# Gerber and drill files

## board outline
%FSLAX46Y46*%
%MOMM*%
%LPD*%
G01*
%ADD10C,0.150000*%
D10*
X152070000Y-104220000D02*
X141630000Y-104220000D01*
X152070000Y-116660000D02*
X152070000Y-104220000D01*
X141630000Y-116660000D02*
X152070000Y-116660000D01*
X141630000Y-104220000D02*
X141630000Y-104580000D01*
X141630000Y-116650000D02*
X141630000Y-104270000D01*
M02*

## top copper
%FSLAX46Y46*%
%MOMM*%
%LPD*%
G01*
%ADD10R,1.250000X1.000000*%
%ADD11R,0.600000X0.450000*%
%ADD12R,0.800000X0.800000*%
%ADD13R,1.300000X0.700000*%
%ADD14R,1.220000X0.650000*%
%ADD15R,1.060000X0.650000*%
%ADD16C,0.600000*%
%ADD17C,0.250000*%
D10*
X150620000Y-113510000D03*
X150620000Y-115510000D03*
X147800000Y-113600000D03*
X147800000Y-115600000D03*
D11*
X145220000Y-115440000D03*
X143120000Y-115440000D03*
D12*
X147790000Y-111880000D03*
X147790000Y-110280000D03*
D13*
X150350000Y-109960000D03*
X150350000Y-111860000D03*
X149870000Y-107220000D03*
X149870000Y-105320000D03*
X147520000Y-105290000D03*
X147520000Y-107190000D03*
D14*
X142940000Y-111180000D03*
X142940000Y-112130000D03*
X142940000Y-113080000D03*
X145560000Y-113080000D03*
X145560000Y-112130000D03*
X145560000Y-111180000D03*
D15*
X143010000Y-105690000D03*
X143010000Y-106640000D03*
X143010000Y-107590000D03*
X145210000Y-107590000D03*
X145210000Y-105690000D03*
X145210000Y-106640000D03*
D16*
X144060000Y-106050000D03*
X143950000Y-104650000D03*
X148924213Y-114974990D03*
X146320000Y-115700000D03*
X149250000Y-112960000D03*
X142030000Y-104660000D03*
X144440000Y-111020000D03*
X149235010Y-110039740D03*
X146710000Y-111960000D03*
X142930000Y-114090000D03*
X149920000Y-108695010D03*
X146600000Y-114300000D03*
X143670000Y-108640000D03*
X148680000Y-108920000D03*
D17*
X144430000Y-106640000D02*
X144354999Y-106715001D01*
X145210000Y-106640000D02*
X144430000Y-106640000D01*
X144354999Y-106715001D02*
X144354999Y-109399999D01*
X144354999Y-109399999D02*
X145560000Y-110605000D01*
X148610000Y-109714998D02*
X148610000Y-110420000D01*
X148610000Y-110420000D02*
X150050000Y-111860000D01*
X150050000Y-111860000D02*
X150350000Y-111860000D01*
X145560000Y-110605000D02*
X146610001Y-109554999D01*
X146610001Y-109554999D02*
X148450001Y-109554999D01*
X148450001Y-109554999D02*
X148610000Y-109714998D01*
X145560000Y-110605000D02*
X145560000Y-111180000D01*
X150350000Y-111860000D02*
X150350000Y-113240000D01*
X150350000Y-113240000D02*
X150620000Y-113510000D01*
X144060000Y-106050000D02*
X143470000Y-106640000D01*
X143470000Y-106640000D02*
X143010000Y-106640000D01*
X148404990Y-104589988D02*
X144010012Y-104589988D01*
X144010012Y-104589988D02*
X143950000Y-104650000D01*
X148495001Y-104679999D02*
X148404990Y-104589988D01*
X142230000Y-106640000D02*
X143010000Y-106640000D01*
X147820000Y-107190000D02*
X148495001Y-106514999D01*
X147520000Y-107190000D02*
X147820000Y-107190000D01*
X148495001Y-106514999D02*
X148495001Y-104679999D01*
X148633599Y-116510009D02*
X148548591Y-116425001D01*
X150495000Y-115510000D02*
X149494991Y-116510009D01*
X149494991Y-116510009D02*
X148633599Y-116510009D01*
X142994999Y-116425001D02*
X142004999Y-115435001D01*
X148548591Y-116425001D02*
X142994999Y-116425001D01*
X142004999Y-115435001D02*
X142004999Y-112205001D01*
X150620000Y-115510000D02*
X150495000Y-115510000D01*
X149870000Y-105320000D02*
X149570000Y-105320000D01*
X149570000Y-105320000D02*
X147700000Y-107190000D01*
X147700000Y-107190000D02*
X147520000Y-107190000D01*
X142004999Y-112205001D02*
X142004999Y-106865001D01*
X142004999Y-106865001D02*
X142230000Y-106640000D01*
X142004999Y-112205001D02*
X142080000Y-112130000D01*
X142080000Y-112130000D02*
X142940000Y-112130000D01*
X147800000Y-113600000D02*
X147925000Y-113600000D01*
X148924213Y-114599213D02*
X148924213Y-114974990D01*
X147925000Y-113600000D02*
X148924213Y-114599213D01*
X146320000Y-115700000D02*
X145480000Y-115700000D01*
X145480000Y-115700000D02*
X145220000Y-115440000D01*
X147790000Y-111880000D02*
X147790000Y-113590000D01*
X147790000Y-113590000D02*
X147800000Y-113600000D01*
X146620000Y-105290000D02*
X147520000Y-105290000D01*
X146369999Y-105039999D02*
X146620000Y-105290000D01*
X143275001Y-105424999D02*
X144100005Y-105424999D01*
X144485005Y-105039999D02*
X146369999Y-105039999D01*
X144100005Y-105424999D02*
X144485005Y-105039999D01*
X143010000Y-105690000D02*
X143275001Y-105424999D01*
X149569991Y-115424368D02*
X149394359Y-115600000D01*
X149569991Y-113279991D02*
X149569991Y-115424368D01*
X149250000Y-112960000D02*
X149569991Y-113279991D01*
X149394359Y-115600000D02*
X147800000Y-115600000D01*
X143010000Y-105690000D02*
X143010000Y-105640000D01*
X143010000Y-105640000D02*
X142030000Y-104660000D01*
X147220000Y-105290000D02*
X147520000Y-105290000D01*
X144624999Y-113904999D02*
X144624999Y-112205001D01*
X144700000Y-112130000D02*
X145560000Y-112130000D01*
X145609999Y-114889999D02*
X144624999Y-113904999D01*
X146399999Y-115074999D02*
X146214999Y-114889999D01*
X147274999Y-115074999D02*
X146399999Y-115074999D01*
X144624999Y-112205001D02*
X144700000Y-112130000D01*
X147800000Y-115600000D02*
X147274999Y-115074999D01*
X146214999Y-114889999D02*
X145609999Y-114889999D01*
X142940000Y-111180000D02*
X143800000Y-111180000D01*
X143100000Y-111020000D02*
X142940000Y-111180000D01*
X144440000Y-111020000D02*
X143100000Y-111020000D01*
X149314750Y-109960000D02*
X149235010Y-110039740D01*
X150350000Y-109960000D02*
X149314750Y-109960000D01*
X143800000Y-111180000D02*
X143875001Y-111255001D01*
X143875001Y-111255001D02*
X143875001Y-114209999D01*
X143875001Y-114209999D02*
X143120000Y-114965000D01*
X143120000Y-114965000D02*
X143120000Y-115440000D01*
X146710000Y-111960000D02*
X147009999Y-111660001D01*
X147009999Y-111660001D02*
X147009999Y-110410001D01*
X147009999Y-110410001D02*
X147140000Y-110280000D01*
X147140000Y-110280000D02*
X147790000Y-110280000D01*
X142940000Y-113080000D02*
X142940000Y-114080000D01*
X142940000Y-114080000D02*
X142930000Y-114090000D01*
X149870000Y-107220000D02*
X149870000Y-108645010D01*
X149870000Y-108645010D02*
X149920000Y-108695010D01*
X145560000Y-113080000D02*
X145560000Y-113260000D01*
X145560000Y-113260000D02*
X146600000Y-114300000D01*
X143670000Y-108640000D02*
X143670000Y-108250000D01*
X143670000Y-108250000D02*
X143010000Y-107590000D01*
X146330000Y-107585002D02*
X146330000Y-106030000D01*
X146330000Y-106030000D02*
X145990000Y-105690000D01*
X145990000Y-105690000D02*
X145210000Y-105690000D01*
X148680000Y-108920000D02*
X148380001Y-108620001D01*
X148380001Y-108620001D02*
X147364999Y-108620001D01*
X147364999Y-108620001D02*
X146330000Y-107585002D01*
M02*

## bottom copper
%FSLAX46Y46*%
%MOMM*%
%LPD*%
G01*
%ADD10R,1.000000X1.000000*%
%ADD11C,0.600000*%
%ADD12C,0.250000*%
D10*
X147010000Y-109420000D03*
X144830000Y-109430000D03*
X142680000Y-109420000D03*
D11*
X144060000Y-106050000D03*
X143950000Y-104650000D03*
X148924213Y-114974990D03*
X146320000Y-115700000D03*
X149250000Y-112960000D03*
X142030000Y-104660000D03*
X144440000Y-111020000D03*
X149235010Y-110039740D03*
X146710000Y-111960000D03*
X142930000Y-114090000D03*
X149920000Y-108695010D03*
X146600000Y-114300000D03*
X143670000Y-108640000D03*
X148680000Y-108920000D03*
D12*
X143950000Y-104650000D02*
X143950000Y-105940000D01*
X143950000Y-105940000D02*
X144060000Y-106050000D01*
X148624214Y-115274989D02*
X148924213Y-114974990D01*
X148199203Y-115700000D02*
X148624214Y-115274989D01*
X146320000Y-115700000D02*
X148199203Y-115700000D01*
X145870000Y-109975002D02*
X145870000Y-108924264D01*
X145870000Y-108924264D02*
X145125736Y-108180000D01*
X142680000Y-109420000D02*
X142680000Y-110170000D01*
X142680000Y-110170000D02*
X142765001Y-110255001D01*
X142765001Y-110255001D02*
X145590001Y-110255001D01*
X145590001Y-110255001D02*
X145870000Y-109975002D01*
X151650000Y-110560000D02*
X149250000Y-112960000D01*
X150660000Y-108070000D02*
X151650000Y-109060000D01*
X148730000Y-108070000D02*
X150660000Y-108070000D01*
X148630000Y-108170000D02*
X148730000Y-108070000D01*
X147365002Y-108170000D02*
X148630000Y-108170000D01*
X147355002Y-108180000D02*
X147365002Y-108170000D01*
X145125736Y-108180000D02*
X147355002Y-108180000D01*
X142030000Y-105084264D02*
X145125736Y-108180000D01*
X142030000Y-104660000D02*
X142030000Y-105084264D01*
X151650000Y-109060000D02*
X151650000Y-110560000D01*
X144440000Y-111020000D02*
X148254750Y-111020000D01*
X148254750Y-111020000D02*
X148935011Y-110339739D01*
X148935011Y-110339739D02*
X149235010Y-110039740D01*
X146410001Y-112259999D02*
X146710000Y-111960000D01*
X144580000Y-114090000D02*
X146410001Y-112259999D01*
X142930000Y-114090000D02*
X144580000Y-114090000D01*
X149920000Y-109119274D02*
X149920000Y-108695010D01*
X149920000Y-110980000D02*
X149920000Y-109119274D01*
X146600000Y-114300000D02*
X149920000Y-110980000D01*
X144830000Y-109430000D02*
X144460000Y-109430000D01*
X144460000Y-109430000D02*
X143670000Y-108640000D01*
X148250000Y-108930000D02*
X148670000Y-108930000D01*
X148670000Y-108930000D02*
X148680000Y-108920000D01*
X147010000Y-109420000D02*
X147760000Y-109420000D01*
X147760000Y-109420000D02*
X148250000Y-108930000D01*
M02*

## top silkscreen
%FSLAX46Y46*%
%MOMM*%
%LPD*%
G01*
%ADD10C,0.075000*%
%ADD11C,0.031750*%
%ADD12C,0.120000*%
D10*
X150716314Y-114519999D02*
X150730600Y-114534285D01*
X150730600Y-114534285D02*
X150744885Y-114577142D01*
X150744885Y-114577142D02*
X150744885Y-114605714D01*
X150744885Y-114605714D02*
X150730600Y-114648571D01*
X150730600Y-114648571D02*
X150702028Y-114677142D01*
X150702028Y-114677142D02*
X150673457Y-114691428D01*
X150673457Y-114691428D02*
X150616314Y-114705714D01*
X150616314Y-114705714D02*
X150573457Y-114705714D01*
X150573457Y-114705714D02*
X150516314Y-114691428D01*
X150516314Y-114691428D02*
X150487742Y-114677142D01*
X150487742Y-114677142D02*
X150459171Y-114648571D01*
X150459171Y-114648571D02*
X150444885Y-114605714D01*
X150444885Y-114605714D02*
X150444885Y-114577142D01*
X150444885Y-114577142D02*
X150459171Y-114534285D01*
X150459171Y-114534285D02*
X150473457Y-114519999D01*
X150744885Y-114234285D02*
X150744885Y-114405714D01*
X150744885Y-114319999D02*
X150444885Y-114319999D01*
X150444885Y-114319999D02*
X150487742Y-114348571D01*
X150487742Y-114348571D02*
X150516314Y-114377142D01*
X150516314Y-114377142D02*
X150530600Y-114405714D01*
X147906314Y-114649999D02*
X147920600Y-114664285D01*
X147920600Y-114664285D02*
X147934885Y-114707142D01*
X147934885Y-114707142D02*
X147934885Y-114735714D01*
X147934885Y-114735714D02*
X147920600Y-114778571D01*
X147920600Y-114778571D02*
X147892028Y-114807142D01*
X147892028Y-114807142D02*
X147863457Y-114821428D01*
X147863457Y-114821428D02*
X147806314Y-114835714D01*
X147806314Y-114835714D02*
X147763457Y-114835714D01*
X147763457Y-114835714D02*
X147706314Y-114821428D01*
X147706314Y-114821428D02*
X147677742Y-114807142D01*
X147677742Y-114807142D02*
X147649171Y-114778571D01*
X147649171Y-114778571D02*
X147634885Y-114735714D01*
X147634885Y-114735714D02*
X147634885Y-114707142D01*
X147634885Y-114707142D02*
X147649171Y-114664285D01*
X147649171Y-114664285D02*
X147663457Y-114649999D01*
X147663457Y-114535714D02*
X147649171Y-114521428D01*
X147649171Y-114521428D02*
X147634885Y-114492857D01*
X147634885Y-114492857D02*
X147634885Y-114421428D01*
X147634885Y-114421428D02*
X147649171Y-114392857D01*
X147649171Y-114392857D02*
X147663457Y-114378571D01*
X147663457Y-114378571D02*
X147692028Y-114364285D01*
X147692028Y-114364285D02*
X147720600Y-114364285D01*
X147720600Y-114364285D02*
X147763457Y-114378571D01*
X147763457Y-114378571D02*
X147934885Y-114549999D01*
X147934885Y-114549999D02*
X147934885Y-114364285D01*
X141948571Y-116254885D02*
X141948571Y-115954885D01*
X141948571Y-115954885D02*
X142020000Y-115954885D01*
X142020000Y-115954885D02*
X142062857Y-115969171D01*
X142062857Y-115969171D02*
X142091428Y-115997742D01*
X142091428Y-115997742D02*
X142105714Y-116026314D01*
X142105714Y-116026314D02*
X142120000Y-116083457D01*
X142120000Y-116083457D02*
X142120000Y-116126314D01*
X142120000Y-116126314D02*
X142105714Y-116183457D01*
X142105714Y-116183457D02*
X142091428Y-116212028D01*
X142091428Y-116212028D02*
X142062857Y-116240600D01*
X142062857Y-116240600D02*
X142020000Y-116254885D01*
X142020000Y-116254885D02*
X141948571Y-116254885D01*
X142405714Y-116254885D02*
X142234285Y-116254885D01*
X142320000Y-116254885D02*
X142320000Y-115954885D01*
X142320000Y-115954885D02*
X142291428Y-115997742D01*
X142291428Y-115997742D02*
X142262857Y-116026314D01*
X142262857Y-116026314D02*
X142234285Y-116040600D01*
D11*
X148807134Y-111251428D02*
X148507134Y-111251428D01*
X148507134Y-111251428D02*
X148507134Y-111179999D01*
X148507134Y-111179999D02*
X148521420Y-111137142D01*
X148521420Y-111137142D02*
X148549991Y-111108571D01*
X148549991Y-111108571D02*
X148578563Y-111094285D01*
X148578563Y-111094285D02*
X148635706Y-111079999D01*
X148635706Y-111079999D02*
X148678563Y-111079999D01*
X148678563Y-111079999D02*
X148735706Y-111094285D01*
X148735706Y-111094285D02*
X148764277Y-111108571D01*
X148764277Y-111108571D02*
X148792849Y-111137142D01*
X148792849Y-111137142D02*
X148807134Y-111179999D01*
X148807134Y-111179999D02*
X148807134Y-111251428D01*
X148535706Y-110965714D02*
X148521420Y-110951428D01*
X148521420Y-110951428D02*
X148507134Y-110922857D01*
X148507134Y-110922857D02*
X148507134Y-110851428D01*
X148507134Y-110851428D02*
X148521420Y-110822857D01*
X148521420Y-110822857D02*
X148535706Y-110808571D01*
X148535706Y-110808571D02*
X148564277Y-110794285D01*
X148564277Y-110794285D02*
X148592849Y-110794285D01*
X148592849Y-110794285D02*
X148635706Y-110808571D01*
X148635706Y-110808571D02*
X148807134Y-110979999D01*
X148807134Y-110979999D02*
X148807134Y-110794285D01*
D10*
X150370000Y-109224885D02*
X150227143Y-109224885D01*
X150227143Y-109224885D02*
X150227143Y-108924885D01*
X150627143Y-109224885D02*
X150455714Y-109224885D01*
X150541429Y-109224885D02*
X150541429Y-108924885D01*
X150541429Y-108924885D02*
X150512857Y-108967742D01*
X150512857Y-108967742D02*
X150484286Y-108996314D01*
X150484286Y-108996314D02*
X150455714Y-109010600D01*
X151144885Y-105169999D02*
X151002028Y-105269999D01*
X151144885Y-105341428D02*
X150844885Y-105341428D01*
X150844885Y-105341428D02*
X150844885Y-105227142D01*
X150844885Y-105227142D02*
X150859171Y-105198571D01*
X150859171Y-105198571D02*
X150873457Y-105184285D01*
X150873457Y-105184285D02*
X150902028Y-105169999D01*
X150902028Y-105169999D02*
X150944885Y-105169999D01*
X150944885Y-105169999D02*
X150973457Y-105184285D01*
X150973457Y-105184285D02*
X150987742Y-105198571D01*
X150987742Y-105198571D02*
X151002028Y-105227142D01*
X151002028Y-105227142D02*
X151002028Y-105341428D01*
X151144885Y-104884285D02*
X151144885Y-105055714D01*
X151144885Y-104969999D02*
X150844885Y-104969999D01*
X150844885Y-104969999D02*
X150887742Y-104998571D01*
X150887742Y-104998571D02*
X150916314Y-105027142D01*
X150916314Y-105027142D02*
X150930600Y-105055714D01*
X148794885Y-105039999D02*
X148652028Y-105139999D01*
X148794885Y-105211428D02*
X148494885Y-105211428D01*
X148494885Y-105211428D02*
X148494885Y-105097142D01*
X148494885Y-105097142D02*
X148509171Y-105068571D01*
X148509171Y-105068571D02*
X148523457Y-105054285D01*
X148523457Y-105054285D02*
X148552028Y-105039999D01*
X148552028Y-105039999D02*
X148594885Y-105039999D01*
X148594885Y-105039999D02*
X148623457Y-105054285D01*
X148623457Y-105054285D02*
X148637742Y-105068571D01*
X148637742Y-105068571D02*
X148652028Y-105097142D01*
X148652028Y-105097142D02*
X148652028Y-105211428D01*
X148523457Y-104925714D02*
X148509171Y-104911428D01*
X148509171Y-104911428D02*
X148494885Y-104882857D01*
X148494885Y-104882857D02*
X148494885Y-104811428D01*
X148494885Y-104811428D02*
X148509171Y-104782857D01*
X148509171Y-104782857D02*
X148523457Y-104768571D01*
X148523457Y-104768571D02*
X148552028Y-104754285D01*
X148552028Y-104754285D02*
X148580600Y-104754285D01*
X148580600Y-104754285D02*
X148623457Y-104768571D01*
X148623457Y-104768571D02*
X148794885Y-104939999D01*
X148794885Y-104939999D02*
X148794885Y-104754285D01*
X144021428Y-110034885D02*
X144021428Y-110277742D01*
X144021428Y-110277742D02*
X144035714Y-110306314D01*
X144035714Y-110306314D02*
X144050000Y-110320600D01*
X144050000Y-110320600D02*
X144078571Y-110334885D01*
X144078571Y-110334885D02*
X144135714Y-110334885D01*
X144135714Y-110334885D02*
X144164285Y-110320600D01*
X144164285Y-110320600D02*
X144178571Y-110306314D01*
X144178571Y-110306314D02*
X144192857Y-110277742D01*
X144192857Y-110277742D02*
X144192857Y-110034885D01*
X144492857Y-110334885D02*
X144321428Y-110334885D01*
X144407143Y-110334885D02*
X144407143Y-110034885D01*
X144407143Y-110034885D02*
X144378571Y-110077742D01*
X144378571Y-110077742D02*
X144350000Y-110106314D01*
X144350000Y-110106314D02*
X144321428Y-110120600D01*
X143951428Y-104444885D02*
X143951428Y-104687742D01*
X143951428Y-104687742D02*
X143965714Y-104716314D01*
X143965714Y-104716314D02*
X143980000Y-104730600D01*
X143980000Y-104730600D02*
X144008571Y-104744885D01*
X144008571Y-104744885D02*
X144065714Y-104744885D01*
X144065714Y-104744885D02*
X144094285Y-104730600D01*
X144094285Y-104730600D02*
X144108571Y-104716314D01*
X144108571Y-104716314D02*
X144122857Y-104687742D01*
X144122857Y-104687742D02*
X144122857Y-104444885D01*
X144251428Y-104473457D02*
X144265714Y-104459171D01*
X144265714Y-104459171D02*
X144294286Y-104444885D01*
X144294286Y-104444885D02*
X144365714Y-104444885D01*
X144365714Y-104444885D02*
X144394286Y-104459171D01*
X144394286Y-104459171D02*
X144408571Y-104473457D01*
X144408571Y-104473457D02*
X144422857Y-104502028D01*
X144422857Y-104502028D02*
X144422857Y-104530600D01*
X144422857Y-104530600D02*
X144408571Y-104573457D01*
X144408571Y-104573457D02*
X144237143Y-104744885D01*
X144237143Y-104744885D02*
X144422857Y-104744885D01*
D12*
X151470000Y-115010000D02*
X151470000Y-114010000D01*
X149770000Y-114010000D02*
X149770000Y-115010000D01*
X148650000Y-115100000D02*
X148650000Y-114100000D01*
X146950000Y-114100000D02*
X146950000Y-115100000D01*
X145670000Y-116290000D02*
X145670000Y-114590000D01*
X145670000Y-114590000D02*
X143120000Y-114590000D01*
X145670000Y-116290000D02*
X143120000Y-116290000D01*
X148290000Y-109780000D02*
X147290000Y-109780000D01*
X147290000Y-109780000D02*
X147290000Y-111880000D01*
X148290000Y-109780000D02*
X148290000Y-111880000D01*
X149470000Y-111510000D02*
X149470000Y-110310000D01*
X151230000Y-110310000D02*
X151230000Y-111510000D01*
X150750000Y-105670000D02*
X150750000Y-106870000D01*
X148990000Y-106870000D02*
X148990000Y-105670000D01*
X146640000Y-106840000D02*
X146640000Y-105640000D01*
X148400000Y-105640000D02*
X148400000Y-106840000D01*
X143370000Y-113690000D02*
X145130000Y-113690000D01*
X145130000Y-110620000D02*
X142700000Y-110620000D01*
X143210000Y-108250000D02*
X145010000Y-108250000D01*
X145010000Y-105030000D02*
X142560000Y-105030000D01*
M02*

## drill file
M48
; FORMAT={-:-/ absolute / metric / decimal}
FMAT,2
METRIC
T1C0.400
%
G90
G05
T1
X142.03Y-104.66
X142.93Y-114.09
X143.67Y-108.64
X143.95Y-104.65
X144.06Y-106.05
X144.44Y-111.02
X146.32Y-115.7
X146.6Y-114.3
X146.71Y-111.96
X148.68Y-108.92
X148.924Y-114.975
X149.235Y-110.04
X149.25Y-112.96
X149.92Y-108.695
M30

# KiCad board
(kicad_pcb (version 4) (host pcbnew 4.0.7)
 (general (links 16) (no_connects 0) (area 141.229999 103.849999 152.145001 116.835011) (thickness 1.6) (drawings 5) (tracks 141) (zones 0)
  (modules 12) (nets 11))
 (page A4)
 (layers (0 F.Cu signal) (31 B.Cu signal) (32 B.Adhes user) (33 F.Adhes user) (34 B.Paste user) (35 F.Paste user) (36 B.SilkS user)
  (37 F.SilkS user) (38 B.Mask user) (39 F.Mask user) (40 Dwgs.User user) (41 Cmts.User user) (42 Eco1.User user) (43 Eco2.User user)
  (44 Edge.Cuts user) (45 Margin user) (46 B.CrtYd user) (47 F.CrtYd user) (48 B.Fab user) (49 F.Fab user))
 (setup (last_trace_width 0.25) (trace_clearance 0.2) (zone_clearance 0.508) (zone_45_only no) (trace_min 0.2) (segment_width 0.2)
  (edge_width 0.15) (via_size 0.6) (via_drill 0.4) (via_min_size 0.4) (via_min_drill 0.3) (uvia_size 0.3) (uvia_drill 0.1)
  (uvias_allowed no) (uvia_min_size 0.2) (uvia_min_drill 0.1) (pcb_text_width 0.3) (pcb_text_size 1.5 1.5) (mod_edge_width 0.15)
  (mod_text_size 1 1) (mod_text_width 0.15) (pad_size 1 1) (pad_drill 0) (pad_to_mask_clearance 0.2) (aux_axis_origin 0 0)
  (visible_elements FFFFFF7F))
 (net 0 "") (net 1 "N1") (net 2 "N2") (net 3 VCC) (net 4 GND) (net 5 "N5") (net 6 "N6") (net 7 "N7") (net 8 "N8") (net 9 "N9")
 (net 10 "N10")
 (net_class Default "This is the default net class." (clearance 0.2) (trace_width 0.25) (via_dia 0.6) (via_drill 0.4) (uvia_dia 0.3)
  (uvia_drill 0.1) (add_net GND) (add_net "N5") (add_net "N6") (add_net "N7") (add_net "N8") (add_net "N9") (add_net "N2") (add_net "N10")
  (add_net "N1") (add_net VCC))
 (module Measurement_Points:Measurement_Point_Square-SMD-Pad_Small (layer B.Cu) (at 147.01 109.42)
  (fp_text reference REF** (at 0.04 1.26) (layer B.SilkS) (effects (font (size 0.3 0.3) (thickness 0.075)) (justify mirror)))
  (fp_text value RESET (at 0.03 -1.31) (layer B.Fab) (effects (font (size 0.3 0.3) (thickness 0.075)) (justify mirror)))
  (pad 1 smd rect (at 0 0) (size 1 1) (layers B.Cu B.Mask) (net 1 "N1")))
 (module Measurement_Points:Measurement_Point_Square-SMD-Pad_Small (layer B.Cu) (at 144.83 109.43)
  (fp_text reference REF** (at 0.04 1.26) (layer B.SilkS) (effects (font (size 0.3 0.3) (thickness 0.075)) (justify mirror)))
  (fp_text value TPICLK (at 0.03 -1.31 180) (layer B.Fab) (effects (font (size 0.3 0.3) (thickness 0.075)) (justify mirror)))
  (pad 1 smd rect (at 0 0) (size 1 1) (layers B.Cu B.Mask) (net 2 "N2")))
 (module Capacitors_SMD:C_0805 (layer F.Cu) (at 150.62 114.51 270)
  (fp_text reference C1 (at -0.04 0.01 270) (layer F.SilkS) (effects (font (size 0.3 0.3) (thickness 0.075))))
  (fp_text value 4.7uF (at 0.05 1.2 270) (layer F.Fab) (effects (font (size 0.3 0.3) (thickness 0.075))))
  (fp_line (start 0.5 -0.85) (end -0.5 -0.85) (layer F.SilkS) (width 0.12))
  (fp_line (start -0.5 0.85) (end 0.5 0.85) (layer F.SilkS) (width 0.12))
  (pad 1 smd rect (at -1 0 270) (size 1 1.25) (layers F.Cu F.Paste F.Mask) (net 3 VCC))
  (pad 2 smd rect (at 1 0 270) (size 1 1.25) (layers F.Cu F.Paste F.Mask) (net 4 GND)))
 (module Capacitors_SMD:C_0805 (layer F.Cu) (at 147.8 114.6 270)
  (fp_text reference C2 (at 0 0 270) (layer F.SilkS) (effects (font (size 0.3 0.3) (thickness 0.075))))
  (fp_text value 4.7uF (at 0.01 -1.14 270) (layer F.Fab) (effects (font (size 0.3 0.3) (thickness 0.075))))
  (fp_line (start 0.5 -0.85) (end -0.5 -0.85) (layer F.SilkS) (width 0.12))
  (fp_line (start -0.5 0.85) (end 0.5 0.85) (layer F.SilkS) (width 0.12))
  (pad 1 smd rect (at -1 0 270) (size 1 1.25) (layers F.Cu F.Paste F.Mask) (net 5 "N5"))
  (pad 2 smd rect (at 1 0 270) (size 1 1.25) (layers F.Cu F.Paste F.Mask) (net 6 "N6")))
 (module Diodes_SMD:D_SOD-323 (layer F.Cu) (at 144.17 115.44 180)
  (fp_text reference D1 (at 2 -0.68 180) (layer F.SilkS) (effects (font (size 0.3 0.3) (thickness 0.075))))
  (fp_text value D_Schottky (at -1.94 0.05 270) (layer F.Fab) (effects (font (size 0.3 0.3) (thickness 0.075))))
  (fp_line (start -1.5 -0.85) (end -1.5 0.85) (layer F.SilkS) (width 0.12))
  (fp_line (start -1.5 0.85) (end 1.05 0.85) (layer F.SilkS) (width 0.12))
  (fp_line (start -1.5 -0.85) (end 1.05 -0.85) (layer F.SilkS) (width 0.12))
  (pad 1 smd rect (at -1.05 0 180) (size 0.6 0.45) (layers F.Cu F.Paste F.Mask) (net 5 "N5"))
  (pad 2 smd rect (at 1.05 0 180) (size 0.6 0.45) (layers F.Cu F.Paste F.Mask) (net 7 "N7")))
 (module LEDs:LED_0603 (layer F.Cu) (at 147.79 111.08 270)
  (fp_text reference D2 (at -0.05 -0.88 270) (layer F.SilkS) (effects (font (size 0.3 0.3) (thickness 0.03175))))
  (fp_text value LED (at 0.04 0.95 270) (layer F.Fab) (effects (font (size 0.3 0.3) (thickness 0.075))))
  (fp_line (start -1.3 -0.5) (end -1.3 0.5) (layer F.SilkS) (width 0.12))
  (fp_line (start -1.3 0.5) (end 0.8 0.5) (layer F.SilkS) (width 0.12))
  (fp_line (start -1.3 -0.5) (end 0.8 -0.5) (layer F.SilkS) (width 0.12))
  (pad 2 smd rect (at 0.8 0 90) (size 0.8 0.8) (layers F.Cu F.Paste F.Mask) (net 5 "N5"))
  (pad 1 smd rect (at -0.8 0 90) (size 0.8 0.8) (layers F.Cu F.Paste F.Mask) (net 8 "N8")))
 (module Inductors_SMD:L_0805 (layer F.Cu) (at 150.35 110.91 270)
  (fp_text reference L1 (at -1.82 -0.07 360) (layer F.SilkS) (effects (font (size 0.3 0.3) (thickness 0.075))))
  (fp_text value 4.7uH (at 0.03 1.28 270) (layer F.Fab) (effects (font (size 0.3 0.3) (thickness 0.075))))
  (fp_line (start 0.6 0.88) (end -0.6 0.88) (layer F.SilkS) (width 0.12))
  (fp_line (start -0.6 -0.88) (end 0.6 -0.88) (layer F.SilkS) (width 0.12))
  (pad 1 smd rect (at -0.95 0 270) (size 0.7 1.3) (layers F.Cu F.Paste F.Mask) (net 7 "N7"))
  (pad 2 smd rect (at 0.95 0 270) (size 0.7 1.3) (layers F.Cu F.Paste F.Mask) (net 3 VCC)))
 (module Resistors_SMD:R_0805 (layer F.Cu) (at 149.87 106.27 90)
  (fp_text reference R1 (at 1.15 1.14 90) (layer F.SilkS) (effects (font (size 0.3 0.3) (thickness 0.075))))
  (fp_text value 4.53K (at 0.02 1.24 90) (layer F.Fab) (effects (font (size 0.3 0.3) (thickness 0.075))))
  (fp_line (start 0.6 0.88) (end -0.6 0.88) (layer F.SilkS) (width 0.12))
  (fp_line (start -0.6 -0.88) (end 0.6 -0.88) (layer F.SilkS) (width 0.12))
  (pad 1 smd rect (at -0.95 0 90) (size 0.7 1.3) (layers F.Cu F.Paste F.Mask) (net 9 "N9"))
  (pad 2 smd rect (at 0.95 0 90) (size 0.7 1.3) (layers F.Cu F.Paste F.Mask) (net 4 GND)))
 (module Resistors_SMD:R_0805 (layer F.Cu) (at 147.52 106.24 270)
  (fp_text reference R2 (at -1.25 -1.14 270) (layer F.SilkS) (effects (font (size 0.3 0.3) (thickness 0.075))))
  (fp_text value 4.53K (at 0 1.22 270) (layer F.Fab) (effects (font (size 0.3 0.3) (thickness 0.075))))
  (fp_line (start 0.6 0.88) (end -0.6 0.88) (layer F.SilkS) (width 0.12))
  (fp_line (start -0.6 -0.88) (end 0.6 -0.88) (layer F.SilkS) (width 0.12))
  (pad 1 smd rect (at -0.95 0 270) (size 0.7 1.3) (layers F.Cu F.Paste F.Mask) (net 6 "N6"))
  (pad 2 smd rect (at 0.95 0 270) (size 0.7 1.3) (layers F.Cu F.Paste F.Mask) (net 4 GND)))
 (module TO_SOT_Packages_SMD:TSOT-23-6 (layer F.Cu) (at 144.25 112.13)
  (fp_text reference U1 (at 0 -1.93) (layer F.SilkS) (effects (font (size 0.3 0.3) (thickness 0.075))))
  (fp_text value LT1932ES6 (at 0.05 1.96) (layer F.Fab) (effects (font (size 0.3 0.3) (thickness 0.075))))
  (fp_line (start -0.88 1.56) (end 0.88 1.56) (layer F.SilkS) (width 0.12))
  (fp_line (start 0.88 -1.51) (end -1.55 -1.51) (layer F.SilkS) (width 0.12))
  (pad 1 smd rect (at -1.31 -0.95) (size 1.22 0.65) (layers F.Cu F.Paste F.Mask) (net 7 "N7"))
  (pad 2 smd rect (at -1.31 0) (size 1.22 0.65) (layers F.Cu F.Paste F.Mask) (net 4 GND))
  (pad 3 smd rect (at -1.31 0.95) (size 1.22 0.65) (layers F.Cu F.Paste F.Mask) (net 8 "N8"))
  (pad 4 smd rect (at 1.31 0.95) (size 1.22 0.65) (layers F.Cu F.Paste F.Mask) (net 9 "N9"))
  (pad 5 smd rect (at 1.31 0) (size 1.22 0.65) (layers F.Cu F.Paste F.Mask) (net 6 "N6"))
  (pad 6 smd rect (at 1.31 -0.95) (size 1.22 0.65) (layers F.Cu F.Paste F.Mask) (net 3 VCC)))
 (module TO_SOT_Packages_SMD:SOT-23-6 (layer F.Cu) (at 144.11 106.64)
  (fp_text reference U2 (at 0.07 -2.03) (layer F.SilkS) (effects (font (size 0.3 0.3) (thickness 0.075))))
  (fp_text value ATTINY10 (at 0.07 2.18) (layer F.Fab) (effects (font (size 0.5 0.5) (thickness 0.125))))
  (fp_line (start -0.9 1.61) (end 0.9 1.61) (layer F.SilkS) (width 0.12))
  (fp_line (start 0.9 -1.61) (end -1.55 -1.61) (layer F.SilkS) (width 0.12))
  (pad 1 smd rect (at -1.1 -0.95) (size 1.06 0.65) (layers F.Cu F.Paste F.Mask) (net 6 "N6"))
  (pad 2 smd rect (at -1.1 0) (size 1.06 0.65) (layers F.Cu F.Paste F.Mask) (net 4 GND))
  (pad 3 smd rect (at -1.1 0.95) (size 1.06 0.65) (layers F.Cu F.Paste F.Mask) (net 2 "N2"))
  (pad 4 smd rect (at 1.1 0.95) (size 1.06 0.65) (layers F.Cu F.Paste F.Mask) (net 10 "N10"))
  (pad 6 smd rect (at 1.1 -0.95) (size 1.06 0.65) (layers F.Cu F.Paste F.Mask) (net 1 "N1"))
  (pad 5 smd rect (at 1.1 0) (size 1.06 0.65) (layers F.Cu F.Paste F.Mask) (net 3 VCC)))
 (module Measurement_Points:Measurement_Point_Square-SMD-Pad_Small (layer B.Cu) (at 142.68 109.42)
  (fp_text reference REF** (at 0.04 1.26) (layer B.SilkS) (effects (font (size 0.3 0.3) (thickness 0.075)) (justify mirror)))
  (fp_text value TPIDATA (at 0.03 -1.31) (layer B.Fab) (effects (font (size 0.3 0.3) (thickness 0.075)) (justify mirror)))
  (pad 1 smd rect (at 0 0) (size 1 1) (layers B.Cu B.Mask) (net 6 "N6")))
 (gr_line (start 152.07 104.22) (end 141.63 104.22) (angle 90) (layer Edge.Cuts) (width 0.15))
 (gr_line (start 152.07 116.66) (end 152.07 104.22) (angle 90) (layer Edge.Cuts) (width 0.15))
 (gr_line (start 141.63 116.66) (end 152.07 116.66) (angle 90) (layer Edge.Cuts) (width 0.15))
 (gr_line (start 141.63 104.22) (end 141.63 104.58) (angle 90) (layer Edge.Cuts) (width 0.15))
 (gr_line (start 141.63 116.65) (end 141.63 104.27) (angle 90) (layer Edge.Cuts) (width 0.15))
 (segment (start 144.43 106.64) (end 144.354999 106.715001) (width 0.25) (layer F.Cu) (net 3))
 (segment (start 145.21 106.64) (end 144.43 106.64) (width 0.25) (layer F.Cu) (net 3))
 (segment (start 144.354999 106.715001) (end 144.354999 109.399999) (width 0.25) (layer F.Cu) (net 3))
 (segment (start 144.354999 109.399999) (end 145.56 110.605) (width 0.25) (layer F.Cu) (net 3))
 (segment (start 148.61 109.714998) (end 148.61 110.42) (width 0.25) (layer F.Cu) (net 3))
 (segment (start 148.61 110.42) (end 150.05 111.86) (width 0.25) (layer F.Cu) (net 3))
 (segment (start 150.05 111.86) (end 150.35 111.86) (width 0.25) (layer F.Cu) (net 3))
 (segment (start 145.56 110.605) (end 146.610001 109.554999) (width 0.25) (layer F.Cu) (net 3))
 (segment (start 146.610001 109.554999) (end 148.450001 109.554999) (width 0.25) (layer F.Cu) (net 3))
 (segment (start 148.450001 109.554999) (end 148.61 109.714998) (width 0.25) (layer F.Cu) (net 3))
 (segment (start 145.56 110.605) (end 145.56 111.18) (width 0.25) (layer F.Cu) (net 3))
 (segment (start 150.35 111.86) (end 150.35 113.24) (width 0.25) (layer F.Cu) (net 3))
 (segment (start 150.35 113.24) (end 150.62 113.51) (width 0.25) (layer F.Cu) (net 3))
 (segment (start 144.06 106.05) (end 143.47 106.64) (width 0.25) (layer F.Cu) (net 4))
 (segment (start 143.47 106.64) (end 143.01 106.64) (width 0.25) (layer F.Cu) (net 4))
 (segment (start 143.95 104.65) (end 143.95 105.94) (width 0.25) (layer B.Cu) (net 4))
 (segment (start 143.95 105.94) (end 144.06 106.05) (width 0.25) (layer B.Cu) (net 4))
 (via (at 144.06 106.05) (size 0.6) (drill 0.4) (layers F.Cu B.Cu) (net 4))
 (segment (start 148.40499 104.589988) (end 144.010012 104.589988) (width 0.25) (layer F.Cu) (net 4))
 (segment (start 144.010012 104.589988) (end 143.95 104.65) (width 0.25) (layer F.Cu) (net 4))
 (segment (start 148.495001 104.679999) (end 148.40499 104.589988) (width 0.25) (layer F.Cu) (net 4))
 (via (at 143.95 104.65) (size 0.6) (drill 0.4) (layers F.Cu B.Cu) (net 4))
 (segment (start 142.23 106.64) (end 143.01 106.64) (width 0.25) (layer F.Cu) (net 4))
 (segment (start 147.82 107.19) (end 148.495001 106.514999) (width 0.25) (layer F.Cu) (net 4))
 (segment (start 147.52 107.19) (end 147.82 107.19) (width 0.25) (layer F.Cu) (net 4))
 (segment (start 148.495001 106.514999) (end 148.495001 104.679999) (width 0.25) (layer F.Cu) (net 4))
 (segment (start 148.633599 116.510009) (end 148.548591 116.425001) (width 0.25) (layer F.Cu) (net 4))
 (segment (start 150.495 115.51) (end 149.494991 116.510009) (width 0.25) (layer F.Cu) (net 4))
 (segment (start 149.494991 116.510009) (end 148.633599 116.510009) (width 0.25) (layer F.Cu) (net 4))
 (segment (start 142.994999 116.425001) (end 142.004999 115.435001) (width 0.25) (layer F.Cu) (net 4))
 (segment (start 148.548591 116.425001) (end 142.994999 116.425001) (width 0.25) (layer F.Cu) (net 4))
 (segment (start 142.004999 115.435001) (end 142.004999 112.205001) (width 0.25) (layer F.Cu) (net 4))
 (segment (start 150.62 115.51) (end 150.495 115.51) (width 0.25) (layer F.Cu) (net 4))
 (segment (start 149.87 105.32) (end 149.57 105.32) (width 0.25) (layer F.Cu) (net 4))
 (segment (start 149.57 105.32) (end 147.7 107.19) (width 0.25) (layer F.Cu) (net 4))
 (segment (start 147.7 107.19) (end 147.52 107.19) (width 0.25) (layer F.Cu) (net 4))
 (segment (start 142.004999 112.205001) (end 142.004999 106.865001) (width 0.25) (layer F.Cu) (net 4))
 (segment (start 142.004999 106.865001) (end 142.23 106.64) (width 0.25) (layer F.Cu) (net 4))
 (segment (start 142.004999 112.205001) (end 142.08 112.13) (width 0.25) (layer F.Cu) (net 4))
 (segment (start 142.08 112.13) (end 142.94 112.13) (width 0.25) (layer F.Cu) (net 4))
 (segment (start 148.624214 115.274989) (end 148.924213 114.97499) (width 0.25) (layer B.Cu) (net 5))
 (segment (start 148.199203 115.7) (end 148.624214 115.274989) (width 0.25) (layer B.Cu) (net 5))
 (segment (start 147.8 113.6) (end 147.925 113.6) (width 0.25) (layer F.Cu) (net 5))
 (segment (start 146.32 115.7) (end 148.199203 115.7) (width 0.25) (layer B.Cu) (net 5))
 (segment (start 148.924213 114.599213) (end 148.924213 114.97499) (width 0.25) (layer F.Cu) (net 5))
 (segment (start 147.925 113.6) (end 148.924213 114.599213) (width 0.25) (layer F.Cu) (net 5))
 (via (at 148.924213 114.97499) (size 0.6) (drill 0.4) (layers F.Cu B.Cu) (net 5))
 (segment (start 146.32 115.7) (end 145.48 115.7) (width 0.25) (layer F.Cu) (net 5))
 (segment (start 145.48 115.7) (end 145.22 115.44) (width 0.25) (layer F.Cu) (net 5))
 (via (at 146.32 115.7) (size 0.6) (drill 0.4) (layers F.Cu B.Cu) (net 5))
 (segment (start 147.79 111.88) (end 147.79 113.59) (width 0.25) (layer F.Cu) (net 5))
 (segment (start 147.79 113.59) (end 147.8 113.6) (width 0.25) (layer F.Cu) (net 5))
 (segment (start 145.87 109.975002) (end 145.87 108.924264) (width 0.25) (layer B.Cu) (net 6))
 (segment (start 145.87 108.924264) (end 145.125736 108.18) (width 0.25) (layer B.Cu) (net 6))
 (segment (start 142.68 109.42) (end 142.68 110.17) (width 0.25) (layer B.Cu) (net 6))
 (segment (start 142.68 110.17) (end 142.765001 110.255001) (width 0.25) (layer B.Cu) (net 6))
 (segment (start 142.765001 110.255001) (end 145.590001 110.255001) (width 0.25) (layer B.Cu) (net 6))
 (segment (start 145.590001 110.255001) (end 145.87 109.975002) (width 0.25) (layer B.Cu) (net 6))
 (segment (start 146.62 105.29) (end 147.52 105.29) (width 0.25) (layer F.Cu) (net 6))
 (segment (start 146.369999 105.039999) (end 146.62 105.29) (width 0.25) (layer F.Cu) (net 6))
 (segment (start 143.275001 105.424999) (end 144.100005 105.424999) (width 0.25) (layer F.Cu) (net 6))
 (segment (start 144.485005 105.039999) (end 146.369999 105.039999) (width 0.25) (layer F.Cu) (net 6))
 (segment (start 144.100005 105.424999) (end 144.485005 105.039999) (width 0.25) (layer F.Cu) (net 6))
 (segment (start 143.01 105.69) (end 143.275001 105.424999) (width 0.25) (layer F.Cu) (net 6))
 (segment (start 151.65 110.56) (end 149.25 112.96) (width 0.25) (layer B.Cu) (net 6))
 (segment (start 150.66 108.07) (end 151.65 109.06) (width 0.25) (layer B.Cu) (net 6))
 (segment (start 148.73 108.07) (end 150.66 108.07) (width 0.25) (layer B.Cu) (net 6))
 (segment (start 148.63 108.17) (end 148.73 108.07) (width 0.25) (layer B.Cu) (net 6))
 (segment (start 147.365002 108.17) (end 148.63 108.17) (width 0.25) (layer B.Cu) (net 6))
 (segment (start 147.355002 108.18) (end 147.365002 108.17) (width 0.25) (layer B.Cu) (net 6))
 (segment (start 145.125736 108.18) (end 147.355002 108.18) (width 0.25) (layer B.Cu) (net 6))
 (segment (start 142.03 105.084264) (end 145.125736 108.18) (width 0.25) (layer B.Cu) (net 6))
 (segment (start 142.03 104.66) (end 142.03 105.084264) (width 0.25) (layer B.Cu) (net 6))
 (segment (start 151.65 109.06) (end 151.65 110.56) (width 0.25) (layer B.Cu) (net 6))
 (segment (start 149.569991 115.424368) (end 149.394359 115.6) (width 0.25) (layer F.Cu) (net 6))
 (segment (start 149.569991 113.279991) (end 149.569991 115.424368) (width 0.25) (layer F.Cu) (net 6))
 (segment (start 149.25 112.96) (end 149.569991 113.279991) (width 0.25) (layer F.Cu) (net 6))
 (segment (start 149.394359 115.6) (end 147.8 115.6) (width 0.25) (layer F.Cu) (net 6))
 (via (at 149.25 112.96) (size 0.6) (drill 0.4) (layers F.Cu B.Cu) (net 6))
 (segment (start 143.01 105.69) (end 143.01 105.64) (width 0.25) (layer F.Cu) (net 6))
 (via (at 142.03 104.66) (size 0.6) (drill 0.4) (layers F.Cu B.Cu) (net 6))
 (segment (start 143.01 105.64) (end 142.03 104.66) (width 0.25) (layer F.Cu) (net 6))
 (segment (start 147.22 105.29) (end 147.52 105.29) (width 0.25) (layer F.Cu) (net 6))
 (segment (start 144.624999 113.904999) (end 144.624999 112.205001) (width 0.25) (layer F.Cu) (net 6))
 (segment (start 144.7 112.13) (end 145.56 112.13) (width 0.25) (layer F.Cu) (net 6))
 (segment (start 145.609999 114.889999) (end 144.624999 113.904999) (width 0.25) (layer F.Cu) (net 6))
 (segment (start 146.399999 115.074999) (end 146.214999 114.889999) (width 0.25) (layer F.Cu) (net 6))
 (segment (start 147.274999 115.074999) (end 146.399999 115.074999) (width 0.25) (layer F.Cu) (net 6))
 (segment (start 144.624999 112.205001) (end 144.7 112.13) (width 0.25) (layer F.Cu) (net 6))
 (segment (start 147.8 115.6) (end 147.274999 115.074999) (width 0.25) (layer F.Cu) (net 6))
 (segment (start 146.214999 114.889999) (end 145.609999 114.889999) (width 0.25) (layer F.Cu) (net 6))
 (segment (start 142.94 111.18) (end 143.8 111.18) (width 0.25) (layer F.Cu) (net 7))
 (segment (start 144.44 111.02) (end 148.25475 111.02) (width 0.25) (layer B.Cu) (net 7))
 (segment (start 148.25475 111.02) (end 148.935011 110.339739) (width 0.25) (layer B.Cu) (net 7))
 (segment (start 143.1 111.02) (end 142.94 111.18) (width 0.25) (layer F.Cu) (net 7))
 (segment (start 144.44 111.02) (end 143.1 111.02) (width 0.25) (layer F.Cu) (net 7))
 (via (at 144.44 111.02) (size 0.6) (drill 0.4) (layers F.Cu B.Cu) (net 7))
 (segment (start 148.935011 110.339739) (end 149.23501 110.03974) (width 0.25) (layer B.Cu) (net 7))
 (segment (start 149.31475 109.96) (end 149.23501 110.03974) (width 0.25) (layer F.Cu) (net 7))
 (segment (start 150.35 109.96) (end 149.31475 109.96) (width 0.25) (layer F.Cu) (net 7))
 (via (at 149.23501 110.03974) (size 0.6) (drill 0.4) (layers F.Cu B.Cu) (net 7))
 (segment (start 143.8 111.18) (end 143.875001 111.255001) (width 0.25) (layer F.Cu) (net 7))
 (segment (start 143.875001 111.255001) (end 143.875001 114.209999) (width 0.25) (layer F.Cu) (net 7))
 (segment (start 143.875001 114.209999) (end 143.12 114.965) (width 0.25) (layer F.Cu) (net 7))
 (segment (start 143.12 114.965) (end 143.12 115.44) (width 0.25) (layer F.Cu) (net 7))
 (segment (start 146.410001 112.259999) (end 146.71 111.96) (width 0.25) (layer B.Cu) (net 8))
 (segment (start 144.58 114.09) (end 146.410001 112.259999) (width 0.25) (layer B.Cu) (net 8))
 (segment (start 142.93 114.09) (end 144.58 114.09) (width 0.25) (layer B.Cu) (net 8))
 (segment (start 146.71 111.96) (end 147.009999 111.660001) (width 0.25) (layer F.Cu) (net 8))
 (segment (start 147.009999 111.660001) (end 147.009999 110.410001) (width 0.25) (layer F.Cu) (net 8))
 (segment (start 147.009999 110.410001) (end 147.14 110.28) (width 0.25) (layer F.Cu) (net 8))
 (segment (start 147.14 110.28) (end 147.79 110.28) (width 0.25) (layer F.Cu) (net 8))
 (via (at 146.71 111.96) (size 0.6) (drill 0.4) (layers F.Cu B.Cu) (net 8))
 (segment (start 142.94 113.08) (end 142.94 114.08) (width 0.25) (layer F.Cu) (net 8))
 (segment (start 142.94 114.08) (end 142.93 114.09) (width 0.25) (layer F.Cu) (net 8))
 (via (at 142.93 114.09) (size 0.6) (drill 0.4) (layers F.Cu B.Cu) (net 8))
 (segment (start 149.87 107.22) (end 149.87 108.64501) (width 0.25) (layer F.Cu) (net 9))
 (segment (start 149.92 109.119274) (end 149.92 108.69501) (width 0.25) (layer B.Cu) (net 9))
 (segment (start 149.92 110.98) (end 149.92 109.119274) (width 0.25) (layer B.Cu) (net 9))
 (segment (start 149.87 108.64501) (end 149.92 108.69501) (width 0.25) (layer F.Cu) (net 9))
 (segment (start 146.6 114.3) (end 149.92 110.98) (width 0.25) (layer B.Cu) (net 9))
 (via (at 149.92 108.69501) (size 0.6) (drill 0.4) (layers F.Cu B.Cu) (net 9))
 (segment (start 145.56 113.08) (end 145.56 113.26) (width 0.25) (layer F.Cu) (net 9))
 (via (at 146.6 114.3) (size 0.6) (drill 0.4) (layers F.Cu B.Cu) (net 9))
 (segment (start 145.56 113.26) (end 146.6 114.3) (width 0.25) (layer F.Cu) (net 9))
 (segment (start 143.67 108.64) (end 143.67 108.25) (width 0.25) (layer F.Cu) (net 2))
 (segment (start 143.67 108.25) (end 143.01 107.59) (width 0.25) (layer F.Cu) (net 2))
 (segment (start 144.83 109.43) (end 144.46 109.43) (width 0.25) (layer B.Cu) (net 2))
 (segment (start 144.46 109.43) (end 143.67 108.64) (width 0.25) (layer B.Cu) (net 2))
 (via (at 143.67 108.64) (size 0.6) (drill 0.4) (layers F.Cu B.Cu) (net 2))
 (segment (start 146.33 107.585002) (end 146.33 106.03) (width 0.25) (layer F.Cu) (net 1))
 (segment (start 146.33 106.03) (end 145.99 105.69) (width 0.25) (layer F.Cu) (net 1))
 (segment (start 145.99 105.69) (end 145.21 105.69) (width 0.25) (layer F.Cu) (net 1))
 (segment (start 148.68 108.92) (end 148.380001 108.620001) (width 0.25) (layer F.Cu) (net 1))
 (segment (start 148.380001 108.620001) (end 147.364999 108.620001) (width 0.25) (layer F.Cu) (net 1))
 (segment (start 147.364999 108.620001) (end 146.33 107.585002) (width 0.25) (layer F.Cu) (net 1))
 (segment (start 148.25 108.93) (end 148.67 108.93) (width 0.25) (layer B.Cu) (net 1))
 (segment (start 148.67 108.93) (end 148.68 108.92) (width 0.25) (layer B.Cu) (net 1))
 (via (at 148.68 108.92) (size 0.6) (drill 0.4) (layers F.Cu B.Cu) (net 1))
 (segment (start 147.01 109.42) (end 147.76 109.42) (width 0.25) (layer B.Cu) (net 1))
 (segment (start 147.76 109.42) (end 148.25 108.93) (width 0.25) (layer B.Cu) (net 1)))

